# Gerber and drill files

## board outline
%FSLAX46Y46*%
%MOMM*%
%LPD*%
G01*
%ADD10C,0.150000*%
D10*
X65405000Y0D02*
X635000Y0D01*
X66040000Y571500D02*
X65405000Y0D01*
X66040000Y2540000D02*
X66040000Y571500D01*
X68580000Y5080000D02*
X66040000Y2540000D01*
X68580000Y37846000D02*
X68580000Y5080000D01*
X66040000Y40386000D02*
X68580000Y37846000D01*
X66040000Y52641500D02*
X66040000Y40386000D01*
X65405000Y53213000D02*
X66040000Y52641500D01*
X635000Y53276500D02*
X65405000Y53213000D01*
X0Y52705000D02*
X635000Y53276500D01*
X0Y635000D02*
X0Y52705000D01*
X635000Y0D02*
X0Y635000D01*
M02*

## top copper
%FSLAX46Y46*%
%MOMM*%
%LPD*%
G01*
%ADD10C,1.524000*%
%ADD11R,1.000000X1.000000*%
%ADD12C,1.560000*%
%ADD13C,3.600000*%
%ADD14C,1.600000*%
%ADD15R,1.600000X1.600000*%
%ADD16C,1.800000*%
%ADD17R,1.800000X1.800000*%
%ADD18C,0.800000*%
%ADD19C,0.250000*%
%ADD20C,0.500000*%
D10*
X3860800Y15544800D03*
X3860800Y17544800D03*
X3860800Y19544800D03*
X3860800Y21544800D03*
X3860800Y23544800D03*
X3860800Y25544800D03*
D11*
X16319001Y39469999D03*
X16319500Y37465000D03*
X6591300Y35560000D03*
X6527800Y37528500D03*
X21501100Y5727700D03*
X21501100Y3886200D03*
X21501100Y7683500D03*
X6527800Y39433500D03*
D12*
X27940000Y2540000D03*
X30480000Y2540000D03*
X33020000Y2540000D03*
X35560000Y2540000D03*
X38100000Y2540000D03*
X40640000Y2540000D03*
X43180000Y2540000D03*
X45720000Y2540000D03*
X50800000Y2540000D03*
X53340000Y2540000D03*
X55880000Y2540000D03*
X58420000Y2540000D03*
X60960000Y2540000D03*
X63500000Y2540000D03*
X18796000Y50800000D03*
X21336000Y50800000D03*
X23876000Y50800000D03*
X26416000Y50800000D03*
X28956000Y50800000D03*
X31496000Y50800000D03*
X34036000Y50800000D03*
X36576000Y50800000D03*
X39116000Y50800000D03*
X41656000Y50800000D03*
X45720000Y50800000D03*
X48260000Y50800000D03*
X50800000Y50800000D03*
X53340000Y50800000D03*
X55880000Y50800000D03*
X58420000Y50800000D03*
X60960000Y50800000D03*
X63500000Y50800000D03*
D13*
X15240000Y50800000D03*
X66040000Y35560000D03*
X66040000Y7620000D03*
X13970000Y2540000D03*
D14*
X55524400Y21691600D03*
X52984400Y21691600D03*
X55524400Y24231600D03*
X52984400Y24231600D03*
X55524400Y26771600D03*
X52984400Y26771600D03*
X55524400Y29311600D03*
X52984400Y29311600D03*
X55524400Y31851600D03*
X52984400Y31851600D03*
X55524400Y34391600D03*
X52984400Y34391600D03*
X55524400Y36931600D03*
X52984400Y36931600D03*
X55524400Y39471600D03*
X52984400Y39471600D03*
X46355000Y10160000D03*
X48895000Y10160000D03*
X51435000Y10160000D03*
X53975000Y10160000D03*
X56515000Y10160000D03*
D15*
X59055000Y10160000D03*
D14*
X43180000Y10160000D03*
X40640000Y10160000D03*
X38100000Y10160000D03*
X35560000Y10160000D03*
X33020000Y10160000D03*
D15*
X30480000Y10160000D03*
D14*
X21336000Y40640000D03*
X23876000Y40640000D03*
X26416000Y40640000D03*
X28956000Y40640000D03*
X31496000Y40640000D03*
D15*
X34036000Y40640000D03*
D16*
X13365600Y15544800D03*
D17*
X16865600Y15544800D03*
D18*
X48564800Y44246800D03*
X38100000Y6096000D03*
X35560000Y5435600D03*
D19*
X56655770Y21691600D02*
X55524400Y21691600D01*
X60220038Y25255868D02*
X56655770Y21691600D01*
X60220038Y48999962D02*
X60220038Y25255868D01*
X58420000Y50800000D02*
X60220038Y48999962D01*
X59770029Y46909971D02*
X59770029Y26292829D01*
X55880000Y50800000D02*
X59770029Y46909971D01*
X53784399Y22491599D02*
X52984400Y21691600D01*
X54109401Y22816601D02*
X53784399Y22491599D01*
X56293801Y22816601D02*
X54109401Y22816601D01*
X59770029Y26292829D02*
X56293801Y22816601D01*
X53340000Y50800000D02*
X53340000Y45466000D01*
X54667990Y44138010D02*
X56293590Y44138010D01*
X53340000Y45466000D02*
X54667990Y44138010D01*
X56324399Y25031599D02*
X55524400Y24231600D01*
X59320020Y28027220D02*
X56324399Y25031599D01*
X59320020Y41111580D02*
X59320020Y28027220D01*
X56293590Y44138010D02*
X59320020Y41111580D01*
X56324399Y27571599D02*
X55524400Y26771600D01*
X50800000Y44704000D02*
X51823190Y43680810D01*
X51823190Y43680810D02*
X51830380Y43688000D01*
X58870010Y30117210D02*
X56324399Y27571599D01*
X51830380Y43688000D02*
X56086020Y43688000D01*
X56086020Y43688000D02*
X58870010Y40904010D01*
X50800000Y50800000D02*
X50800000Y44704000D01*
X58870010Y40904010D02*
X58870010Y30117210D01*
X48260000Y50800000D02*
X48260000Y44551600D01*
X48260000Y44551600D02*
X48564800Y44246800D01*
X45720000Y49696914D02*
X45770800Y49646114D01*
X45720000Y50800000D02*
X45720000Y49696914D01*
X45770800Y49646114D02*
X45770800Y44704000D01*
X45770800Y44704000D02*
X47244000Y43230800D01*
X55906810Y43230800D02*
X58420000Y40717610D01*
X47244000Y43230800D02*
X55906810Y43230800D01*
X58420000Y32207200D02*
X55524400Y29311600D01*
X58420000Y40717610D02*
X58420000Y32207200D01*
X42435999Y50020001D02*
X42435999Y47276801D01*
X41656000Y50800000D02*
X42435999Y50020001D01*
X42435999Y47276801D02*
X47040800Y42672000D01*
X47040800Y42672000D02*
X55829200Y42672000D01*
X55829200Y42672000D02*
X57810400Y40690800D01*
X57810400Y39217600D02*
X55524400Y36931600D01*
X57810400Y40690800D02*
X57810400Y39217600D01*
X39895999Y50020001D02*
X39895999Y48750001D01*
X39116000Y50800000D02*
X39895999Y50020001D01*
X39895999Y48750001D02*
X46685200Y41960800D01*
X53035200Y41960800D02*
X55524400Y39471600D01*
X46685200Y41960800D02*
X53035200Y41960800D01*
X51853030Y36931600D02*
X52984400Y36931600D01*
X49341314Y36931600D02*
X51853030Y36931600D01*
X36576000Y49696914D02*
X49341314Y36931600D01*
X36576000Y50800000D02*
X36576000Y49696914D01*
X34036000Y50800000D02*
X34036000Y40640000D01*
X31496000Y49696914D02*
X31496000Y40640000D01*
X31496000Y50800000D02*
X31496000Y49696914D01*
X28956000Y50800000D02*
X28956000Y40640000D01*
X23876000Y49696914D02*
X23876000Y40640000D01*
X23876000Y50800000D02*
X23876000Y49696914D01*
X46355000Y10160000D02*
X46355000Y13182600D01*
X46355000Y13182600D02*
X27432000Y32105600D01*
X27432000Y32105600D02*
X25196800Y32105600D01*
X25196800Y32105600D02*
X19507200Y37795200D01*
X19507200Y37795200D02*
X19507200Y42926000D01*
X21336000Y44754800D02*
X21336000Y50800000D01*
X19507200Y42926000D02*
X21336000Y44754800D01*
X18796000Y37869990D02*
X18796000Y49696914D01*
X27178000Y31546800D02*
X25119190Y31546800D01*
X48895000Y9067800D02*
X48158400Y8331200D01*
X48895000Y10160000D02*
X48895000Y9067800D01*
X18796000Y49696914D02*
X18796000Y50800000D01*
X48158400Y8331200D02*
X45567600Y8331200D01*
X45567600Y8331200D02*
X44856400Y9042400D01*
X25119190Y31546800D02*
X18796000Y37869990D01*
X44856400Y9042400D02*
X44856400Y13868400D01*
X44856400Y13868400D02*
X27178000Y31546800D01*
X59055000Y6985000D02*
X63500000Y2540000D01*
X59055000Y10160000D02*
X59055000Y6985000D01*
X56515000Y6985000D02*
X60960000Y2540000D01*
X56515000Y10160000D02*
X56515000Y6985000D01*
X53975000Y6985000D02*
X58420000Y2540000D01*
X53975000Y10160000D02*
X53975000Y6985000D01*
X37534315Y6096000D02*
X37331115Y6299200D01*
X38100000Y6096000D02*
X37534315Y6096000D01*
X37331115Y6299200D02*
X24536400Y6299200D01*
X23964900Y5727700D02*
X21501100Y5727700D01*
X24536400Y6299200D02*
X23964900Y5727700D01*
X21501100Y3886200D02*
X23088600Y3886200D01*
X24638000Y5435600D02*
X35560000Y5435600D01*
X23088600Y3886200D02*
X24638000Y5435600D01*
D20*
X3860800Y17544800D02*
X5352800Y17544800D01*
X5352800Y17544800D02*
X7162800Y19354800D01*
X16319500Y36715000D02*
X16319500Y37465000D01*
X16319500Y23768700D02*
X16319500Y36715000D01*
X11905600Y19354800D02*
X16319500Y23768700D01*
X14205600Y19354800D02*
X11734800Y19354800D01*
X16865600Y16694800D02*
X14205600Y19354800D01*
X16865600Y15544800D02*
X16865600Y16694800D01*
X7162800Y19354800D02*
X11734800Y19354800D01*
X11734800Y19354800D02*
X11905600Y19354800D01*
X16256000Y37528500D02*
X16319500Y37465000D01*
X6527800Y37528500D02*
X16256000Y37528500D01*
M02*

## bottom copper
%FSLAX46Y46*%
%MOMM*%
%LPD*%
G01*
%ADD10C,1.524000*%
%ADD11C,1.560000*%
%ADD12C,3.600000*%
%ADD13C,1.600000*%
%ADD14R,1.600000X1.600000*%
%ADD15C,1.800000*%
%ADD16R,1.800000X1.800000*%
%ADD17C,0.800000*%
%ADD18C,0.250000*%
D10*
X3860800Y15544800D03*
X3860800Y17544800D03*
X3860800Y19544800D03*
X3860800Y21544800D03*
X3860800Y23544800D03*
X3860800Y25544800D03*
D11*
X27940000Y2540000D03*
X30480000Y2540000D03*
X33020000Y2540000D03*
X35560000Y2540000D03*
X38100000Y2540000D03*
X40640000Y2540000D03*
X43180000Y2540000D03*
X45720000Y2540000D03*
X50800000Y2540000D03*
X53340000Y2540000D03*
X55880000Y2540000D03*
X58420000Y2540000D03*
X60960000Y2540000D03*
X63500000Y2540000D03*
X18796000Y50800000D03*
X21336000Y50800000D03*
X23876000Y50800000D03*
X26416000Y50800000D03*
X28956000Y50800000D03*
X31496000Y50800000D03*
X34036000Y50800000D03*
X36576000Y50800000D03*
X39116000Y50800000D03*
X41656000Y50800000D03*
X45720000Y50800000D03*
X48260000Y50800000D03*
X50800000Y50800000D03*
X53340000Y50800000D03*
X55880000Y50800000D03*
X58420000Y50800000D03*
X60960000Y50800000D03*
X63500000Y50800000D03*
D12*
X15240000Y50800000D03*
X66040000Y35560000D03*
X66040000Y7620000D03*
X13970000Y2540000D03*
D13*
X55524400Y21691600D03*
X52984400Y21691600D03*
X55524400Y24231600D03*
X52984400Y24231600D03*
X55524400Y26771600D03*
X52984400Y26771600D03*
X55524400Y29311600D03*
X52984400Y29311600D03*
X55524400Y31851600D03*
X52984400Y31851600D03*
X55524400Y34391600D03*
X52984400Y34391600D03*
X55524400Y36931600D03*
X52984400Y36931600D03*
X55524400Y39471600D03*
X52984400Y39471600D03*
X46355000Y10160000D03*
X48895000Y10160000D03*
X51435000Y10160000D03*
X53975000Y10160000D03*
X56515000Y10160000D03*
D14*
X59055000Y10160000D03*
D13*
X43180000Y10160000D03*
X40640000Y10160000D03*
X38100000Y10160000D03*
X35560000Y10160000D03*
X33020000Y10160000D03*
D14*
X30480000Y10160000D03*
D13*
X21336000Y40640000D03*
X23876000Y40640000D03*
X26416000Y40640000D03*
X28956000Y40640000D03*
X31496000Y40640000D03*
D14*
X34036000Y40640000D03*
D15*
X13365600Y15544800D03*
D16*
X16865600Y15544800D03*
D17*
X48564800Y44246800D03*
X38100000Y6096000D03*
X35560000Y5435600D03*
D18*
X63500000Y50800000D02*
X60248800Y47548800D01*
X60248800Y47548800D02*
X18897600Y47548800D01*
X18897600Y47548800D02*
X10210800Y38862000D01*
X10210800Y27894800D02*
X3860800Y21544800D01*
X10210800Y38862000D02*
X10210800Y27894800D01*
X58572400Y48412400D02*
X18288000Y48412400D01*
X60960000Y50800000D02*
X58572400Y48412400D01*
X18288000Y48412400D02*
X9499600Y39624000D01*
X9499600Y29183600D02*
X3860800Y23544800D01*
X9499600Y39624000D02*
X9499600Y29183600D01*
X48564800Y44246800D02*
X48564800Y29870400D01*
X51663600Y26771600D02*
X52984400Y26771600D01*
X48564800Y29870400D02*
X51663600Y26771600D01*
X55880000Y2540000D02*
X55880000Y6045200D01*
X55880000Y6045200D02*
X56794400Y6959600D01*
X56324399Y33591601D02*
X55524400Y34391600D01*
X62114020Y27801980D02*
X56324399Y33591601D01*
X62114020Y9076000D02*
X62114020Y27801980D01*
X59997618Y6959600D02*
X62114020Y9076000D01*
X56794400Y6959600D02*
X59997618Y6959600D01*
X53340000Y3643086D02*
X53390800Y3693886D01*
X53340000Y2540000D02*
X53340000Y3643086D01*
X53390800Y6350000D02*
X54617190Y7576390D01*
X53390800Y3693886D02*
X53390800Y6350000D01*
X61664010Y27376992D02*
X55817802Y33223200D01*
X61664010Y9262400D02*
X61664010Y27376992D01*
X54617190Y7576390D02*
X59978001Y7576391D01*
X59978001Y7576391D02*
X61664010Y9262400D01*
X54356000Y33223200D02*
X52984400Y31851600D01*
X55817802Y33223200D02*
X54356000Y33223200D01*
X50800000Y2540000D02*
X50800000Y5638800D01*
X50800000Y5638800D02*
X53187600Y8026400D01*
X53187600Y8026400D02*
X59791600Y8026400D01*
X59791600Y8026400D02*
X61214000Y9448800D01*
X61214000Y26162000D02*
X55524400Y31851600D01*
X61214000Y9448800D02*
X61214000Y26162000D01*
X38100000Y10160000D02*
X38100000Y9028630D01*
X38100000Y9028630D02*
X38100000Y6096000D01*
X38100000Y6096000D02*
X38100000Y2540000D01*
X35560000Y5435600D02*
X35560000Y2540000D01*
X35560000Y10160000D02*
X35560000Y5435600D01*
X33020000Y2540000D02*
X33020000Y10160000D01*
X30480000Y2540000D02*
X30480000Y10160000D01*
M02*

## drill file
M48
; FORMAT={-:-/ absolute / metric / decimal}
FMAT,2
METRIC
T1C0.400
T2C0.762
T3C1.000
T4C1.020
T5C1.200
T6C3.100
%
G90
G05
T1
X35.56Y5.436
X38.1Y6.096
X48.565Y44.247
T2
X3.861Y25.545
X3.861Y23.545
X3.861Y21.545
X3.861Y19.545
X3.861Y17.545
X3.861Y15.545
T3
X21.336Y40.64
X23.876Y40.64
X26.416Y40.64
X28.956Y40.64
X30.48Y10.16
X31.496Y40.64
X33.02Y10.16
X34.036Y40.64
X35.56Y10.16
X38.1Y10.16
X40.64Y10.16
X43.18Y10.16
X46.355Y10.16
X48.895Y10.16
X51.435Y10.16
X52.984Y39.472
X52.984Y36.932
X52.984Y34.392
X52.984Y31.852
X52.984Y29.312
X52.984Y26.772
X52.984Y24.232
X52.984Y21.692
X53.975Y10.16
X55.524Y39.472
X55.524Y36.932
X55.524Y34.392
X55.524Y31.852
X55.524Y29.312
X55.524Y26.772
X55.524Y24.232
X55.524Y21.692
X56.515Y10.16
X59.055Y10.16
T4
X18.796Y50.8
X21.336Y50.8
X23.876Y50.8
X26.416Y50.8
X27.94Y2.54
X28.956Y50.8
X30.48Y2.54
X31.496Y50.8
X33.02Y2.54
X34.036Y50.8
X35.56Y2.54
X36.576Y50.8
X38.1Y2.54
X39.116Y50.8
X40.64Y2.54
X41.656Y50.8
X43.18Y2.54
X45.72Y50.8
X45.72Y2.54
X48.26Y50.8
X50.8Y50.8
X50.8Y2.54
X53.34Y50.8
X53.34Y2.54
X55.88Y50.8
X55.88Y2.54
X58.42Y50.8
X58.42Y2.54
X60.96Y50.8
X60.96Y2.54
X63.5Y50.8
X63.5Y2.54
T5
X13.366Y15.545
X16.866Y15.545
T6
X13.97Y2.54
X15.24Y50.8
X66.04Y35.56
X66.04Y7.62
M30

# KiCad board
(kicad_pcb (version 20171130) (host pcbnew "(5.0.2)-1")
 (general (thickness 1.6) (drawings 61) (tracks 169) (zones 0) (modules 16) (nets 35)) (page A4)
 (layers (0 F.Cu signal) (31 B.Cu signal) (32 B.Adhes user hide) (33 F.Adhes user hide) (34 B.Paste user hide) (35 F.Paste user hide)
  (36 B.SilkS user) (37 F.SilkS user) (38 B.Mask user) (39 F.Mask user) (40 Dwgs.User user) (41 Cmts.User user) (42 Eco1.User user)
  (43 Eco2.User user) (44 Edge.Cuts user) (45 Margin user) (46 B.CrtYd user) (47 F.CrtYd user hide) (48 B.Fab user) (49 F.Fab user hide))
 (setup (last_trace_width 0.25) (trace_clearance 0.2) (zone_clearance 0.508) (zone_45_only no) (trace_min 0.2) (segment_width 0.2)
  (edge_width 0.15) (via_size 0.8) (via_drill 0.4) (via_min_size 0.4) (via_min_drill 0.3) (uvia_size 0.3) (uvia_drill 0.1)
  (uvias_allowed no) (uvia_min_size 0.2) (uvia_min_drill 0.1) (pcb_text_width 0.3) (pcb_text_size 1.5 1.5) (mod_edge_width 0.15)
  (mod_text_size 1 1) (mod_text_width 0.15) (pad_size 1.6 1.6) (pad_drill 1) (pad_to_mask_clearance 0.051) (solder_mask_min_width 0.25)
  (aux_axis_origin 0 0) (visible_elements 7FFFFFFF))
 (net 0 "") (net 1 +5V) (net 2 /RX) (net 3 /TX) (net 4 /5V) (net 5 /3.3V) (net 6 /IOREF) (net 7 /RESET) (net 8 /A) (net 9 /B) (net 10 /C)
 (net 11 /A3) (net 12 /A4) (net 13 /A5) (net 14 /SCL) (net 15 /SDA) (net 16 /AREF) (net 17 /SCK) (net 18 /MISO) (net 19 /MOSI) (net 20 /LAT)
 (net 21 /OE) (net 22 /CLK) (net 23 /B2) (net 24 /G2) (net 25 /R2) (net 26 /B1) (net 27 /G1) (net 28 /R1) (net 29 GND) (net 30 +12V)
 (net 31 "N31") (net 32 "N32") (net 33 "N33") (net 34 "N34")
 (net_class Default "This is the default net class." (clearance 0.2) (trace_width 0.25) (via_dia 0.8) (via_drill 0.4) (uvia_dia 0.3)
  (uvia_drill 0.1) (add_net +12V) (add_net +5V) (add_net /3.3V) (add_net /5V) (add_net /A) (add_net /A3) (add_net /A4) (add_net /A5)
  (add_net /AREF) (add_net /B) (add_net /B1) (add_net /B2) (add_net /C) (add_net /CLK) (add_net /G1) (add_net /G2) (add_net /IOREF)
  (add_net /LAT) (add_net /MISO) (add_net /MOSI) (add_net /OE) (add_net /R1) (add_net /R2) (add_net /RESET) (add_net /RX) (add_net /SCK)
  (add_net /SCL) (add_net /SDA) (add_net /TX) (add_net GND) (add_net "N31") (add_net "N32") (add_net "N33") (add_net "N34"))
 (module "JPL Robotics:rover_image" (layer F.Cu) (at 38.4556 -27.7368 90)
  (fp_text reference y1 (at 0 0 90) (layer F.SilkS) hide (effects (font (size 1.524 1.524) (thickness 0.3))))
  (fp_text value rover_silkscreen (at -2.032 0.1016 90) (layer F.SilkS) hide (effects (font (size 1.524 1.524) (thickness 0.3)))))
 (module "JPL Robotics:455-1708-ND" (layer F.Cu) (at 3.8608 -15.5448 90)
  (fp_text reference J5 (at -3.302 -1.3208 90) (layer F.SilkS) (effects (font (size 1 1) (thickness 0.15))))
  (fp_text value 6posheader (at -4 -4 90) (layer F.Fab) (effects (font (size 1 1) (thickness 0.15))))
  (pad 1 thru_hole circle (at 0 0 90) (size 1.524 1.524) (drill 0.762) (layers *.Cu *.Mask))
  (pad 2 thru_hole circle (at 2 0 90) (size 1.524 1.524) (drill 0.762) (layers *.Cu *.Mask) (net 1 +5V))
  (pad 3 thru_hole circle (at 4 0 90) (size 1.524 1.524) (drill 0.762) (layers *.Cu *.Mask))
  (pad 4 thru_hole circle (at 6 0 90) (size 1.524 1.524) (drill 0.762) (layers *.Cu *.Mask) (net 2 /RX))
  (pad 5 thru_hole circle (at 8 0 90) (size 1.524 1.524) (drill 0.762) (layers *.Cu *.Mask) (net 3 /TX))
  (pad 6 thru_hole circle (at 10 0 90) (size 1.524 1.524) (drill 0.762) (layers *.Cu *.Mask)))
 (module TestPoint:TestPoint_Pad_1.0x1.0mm (layer F.Cu) (at 16.319001 -39.469999)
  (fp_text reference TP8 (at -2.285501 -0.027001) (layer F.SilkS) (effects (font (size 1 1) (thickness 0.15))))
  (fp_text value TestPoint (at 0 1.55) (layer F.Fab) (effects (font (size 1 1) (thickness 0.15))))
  (pad 1 smd rect (at 0 0) (size 1 1) (layers F.Cu F.Mask)))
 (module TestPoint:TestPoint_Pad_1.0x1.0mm (layer F.Cu) (at 16.3195 -37.465)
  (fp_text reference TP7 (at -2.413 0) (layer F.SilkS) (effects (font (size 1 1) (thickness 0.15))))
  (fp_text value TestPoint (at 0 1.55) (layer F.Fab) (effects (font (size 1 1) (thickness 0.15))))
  (pad 1 smd rect (at 0 0) (size 1 1) (layers F.Cu F.Mask) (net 1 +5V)))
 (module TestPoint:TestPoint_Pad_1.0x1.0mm (layer F.Cu) (at 6.5913 -35.56)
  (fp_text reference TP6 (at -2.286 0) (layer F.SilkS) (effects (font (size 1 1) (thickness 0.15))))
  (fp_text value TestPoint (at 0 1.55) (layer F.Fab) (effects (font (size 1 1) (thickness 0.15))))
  (pad 1 smd rect (at 0 0) (size 1 1) (layers F.Cu F.Mask)))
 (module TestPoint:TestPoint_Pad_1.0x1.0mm (layer F.Cu) (at 6.5278 -37.5285)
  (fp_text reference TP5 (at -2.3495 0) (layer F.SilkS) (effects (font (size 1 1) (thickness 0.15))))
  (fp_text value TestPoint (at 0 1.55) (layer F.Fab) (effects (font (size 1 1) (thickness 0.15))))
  (pad 1 smd rect (at 0 0) (size 1 1) (layers F.Cu F.Mask) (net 1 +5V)))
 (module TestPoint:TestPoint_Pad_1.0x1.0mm (layer F.Cu) (at 21.5011 -5.7277 90)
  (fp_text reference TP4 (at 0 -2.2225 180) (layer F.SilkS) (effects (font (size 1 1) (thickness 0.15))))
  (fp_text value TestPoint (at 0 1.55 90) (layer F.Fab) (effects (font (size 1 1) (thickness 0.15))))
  (pad 1 smd rect (at 0 0 90) (size 1 1) (layers F.Cu F.Mask) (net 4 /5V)))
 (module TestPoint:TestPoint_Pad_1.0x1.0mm (layer F.Cu) (at 21.5011 -3.8862 90)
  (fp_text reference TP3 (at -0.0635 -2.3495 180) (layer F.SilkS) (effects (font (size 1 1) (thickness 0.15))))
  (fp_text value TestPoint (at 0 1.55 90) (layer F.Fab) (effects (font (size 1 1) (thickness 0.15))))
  (pad 1 smd rect (at 0 0 90) (size 1 1) (layers F.Cu F.Mask) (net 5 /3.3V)))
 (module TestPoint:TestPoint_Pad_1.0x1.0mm (layer F.Cu) (at 21.5011 -7.6835 90)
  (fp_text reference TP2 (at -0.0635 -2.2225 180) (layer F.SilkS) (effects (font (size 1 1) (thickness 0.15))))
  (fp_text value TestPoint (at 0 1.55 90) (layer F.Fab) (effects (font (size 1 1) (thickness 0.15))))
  (pad 1 smd rect (at 0 0 90) (size 1 1) (layers F.Cu F.Mask)))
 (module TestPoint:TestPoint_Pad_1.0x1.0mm (layer F.Cu) (at 6.5278 -39.4335)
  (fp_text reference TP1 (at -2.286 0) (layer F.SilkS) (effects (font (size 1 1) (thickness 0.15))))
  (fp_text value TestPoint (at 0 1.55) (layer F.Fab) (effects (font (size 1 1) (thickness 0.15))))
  (pad 1 smd rect (at 0 0) (size 1 1) (layers F.Cu F.Mask)))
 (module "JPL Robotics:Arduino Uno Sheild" (layer F.Cu) (at 0 0)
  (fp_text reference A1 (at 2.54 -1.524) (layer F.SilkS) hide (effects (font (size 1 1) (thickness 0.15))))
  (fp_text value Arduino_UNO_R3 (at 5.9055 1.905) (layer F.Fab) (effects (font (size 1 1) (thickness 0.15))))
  (pad 31 thru_hole circle (at 27.94 -2.54) (size 1.56 1.56) (drill 1.02) (layers *.Cu *.Mask))
  (pad 20 thru_hole circle (at 30.48 -2.54) (size 1.56 1.56) (drill 1.02) (layers *.Cu *.Mask) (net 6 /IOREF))
  (pad 21 thru_hole circle (at 33.02 -2.54) (size 1.56 1.56) (drill 1.02) (layers *.Cu *.Mask) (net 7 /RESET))
  (pad 22 thru_hole circle (at 35.56 -2.54) (size 1.56 1.56) (drill 1.02) (layers *.Cu *.Mask) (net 5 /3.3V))
  (pad 23 thru_hole circle (at 38.1 -2.54) (size 1.56 1.56) (drill 1.02) (layers *.Cu *.Mask) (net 4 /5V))
  (pad 24 thru_hole circle (at 40.64 -2.54) (size 1.56 1.56) (drill 1.02) (layers *.Cu *.Mask))
  (pad 25 thru_hole circle (at 43.18 -2.54) (size 1.56 1.56) (drill 1.02) (layers *.Cu *.Mask))
  (pad 26 thru_hole circle (at 45.72 -2.54) (size 1.56 1.56) (drill 1.02) (layers *.Cu *.Mask))
  (pad 14 thru_hole circle (at 50.8 -2.54) (size 1.56 1.56) (drill 1.02) (layers *.Cu *.Mask) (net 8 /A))
  (pad 15 thru_hole circle (at 53.34 -2.54) (size 1.56 1.56) (drill 1.02) (layers *.Cu *.Mask) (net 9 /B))
  (pad 16 thru_hole circle (at 55.88 -2.54) (size 1.56 1.56) (drill 1.02) (layers *.Cu *.Mask) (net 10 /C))
  (pad 17 thru_hole circle (at 58.42 -2.54) (size 1.56 1.56) (drill 1.02) (layers *.Cu *.Mask) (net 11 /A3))
  (pad 18 thru_hole circle (at 60.96 -2.54) (size 1.56 1.56) (drill 1.02) (layers *.Cu *.Mask) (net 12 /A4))
  (pad 19 thru_hole circle (at 63.5 -2.54) (size 1.56 1.56) (drill 1.02) (layers *.Cu *.Mask) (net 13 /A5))
  (pad 30 thru_hole circle (at 18.796 -50.8) (size 1.56 1.56) (drill 1.02) (layers *.Cu *.Mask) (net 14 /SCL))
  (pad 29 thru_hole circle (at 21.336 -50.8) (size 1.56 1.56) (drill 1.02) (layers *.Cu *.Mask) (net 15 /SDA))
  (pad 28 thru_hole circle (at 23.876 -50.8) (size 1.56 1.56) (drill 1.02) (layers *.Cu *.Mask) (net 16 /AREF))
  (pad 27 thru_hole circle (at 26.416 -50.8) (size 1.56 1.56) (drill 1.02) (layers *.Cu *.Mask))
  (pad 13 thru_hole circle (at 28.956 -50.8) (size 1.56 1.56) (drill 1.02) (layers *.Cu *.Mask) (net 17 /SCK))
  (pad 12 thru_hole circle (at 31.496 -50.8) (size 1.56 1.56) (drill 1.02) (layers *.Cu *.Mask) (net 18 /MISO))
  (pad 11 thru_hole circle (at 34.036 -50.8) (size 1.56 1.56) (drill 1.02) (layers *.Cu *.Mask) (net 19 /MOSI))
  (pad 10 thru_hole circle (at 36.576 -50.8) (size 1.56 1.56) (drill 1.02) (layers *.Cu *.Mask) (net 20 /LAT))
  (pad 9 thru_hole circle (at 39.116 -50.8) (size 1.56 1.56) (drill 1.02) (layers *.Cu *.Mask) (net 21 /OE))
  (pad 8 thru_hole circle (at 41.656 -50.8) (size 1.56 1.56) (drill 1.02) (layers *.Cu *.Mask) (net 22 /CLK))
  (pad 7 thru_hole circle (at 45.72 -50.8) (size 1.56 1.56) (drill 1.02) (layers *.Cu *.Mask) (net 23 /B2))
  (pad 6 thru_hole circle (at 48.26 -50.8) (size 1.56 1.56) (drill 1.02) (layers *.Cu *.Mask) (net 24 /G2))
  (pad 5 thru_hole circle (at 50.8 -50.8) (size 1.56 1.56) (drill 1.02) (layers *.Cu *.Mask) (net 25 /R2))
  (pad 4 thru_hole circle (at 53.34 -50.8) (size 1.56 1.56) (drill 1.02) (layers *.Cu *.Mask) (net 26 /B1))
  (pad 3 thru_hole circle (at 55.88 -50.8) (size 1.56 1.56) (drill 1.02) (layers *.Cu *.Mask) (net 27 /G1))
  (pad 2 thru_hole circle (at 58.42 -50.8) (size 1.56 1.56) (drill 1.02) (layers *.Cu *.Mask) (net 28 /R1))
  (pad 1 thru_hole circle (at 60.96 -50.8) (size 1.56 1.56) (drill 1.02) (layers *.Cu *.Mask) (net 3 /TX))
  (pad 0 thru_hole circle (at 63.5 -50.8) (size 1.56 1.56) (drill 1.02) (layers *.Cu *.Mask) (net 2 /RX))
  (pad "" np_thru_hole circle (at 15.24 -50.8) (size 3.6 3.6) (drill 3.1) (layers *.Cu *.Mask))
  (pad "" np_thru_hole circle (at 66.04 -35.56) (size 3.6 3.6) (drill 3.1) (layers *.Cu *.Mask))
  (pad "" np_thru_hole circle (at 66.04 -7.62) (size 3.6 3.6) (drill 3.1) (layers *.Cu *.Mask))
  (pad "" np_thru_hole circle (at 13.97 -2.54) (size 3.6 3.6) (drill 3.1) (layers *.Cu *.Mask)))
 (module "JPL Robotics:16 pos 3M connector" (layer F.Cu) (at 54.2544 -30.5816 90)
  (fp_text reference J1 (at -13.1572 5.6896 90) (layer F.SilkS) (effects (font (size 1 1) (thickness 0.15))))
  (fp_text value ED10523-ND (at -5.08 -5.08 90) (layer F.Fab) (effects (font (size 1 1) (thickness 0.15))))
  (pad 1 thru_hole circle (at -8.89 1.27 90) (size 1.6 1.6) (drill 1) (layers *.Cu *.Mask) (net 28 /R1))
  (pad 2 thru_hole circle (at -8.89 -1.27 90) (size 1.6 1.6) (drill 1) (layers *.Cu *.Mask) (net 27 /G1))
  (pad 3 thru_hole circle (at -6.35 1.27 90) (size 1.6 1.6) (drill 1) (layers *.Cu *.Mask) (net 26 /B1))
  (pad 4 thru_hole circle (at -6.35 -1.27 90) (size 1.6 1.6) (drill 1) (layers *.Cu *.Mask))
  (pad 5 thru_hole circle (at -3.81 1.27 90) (size 1.6 1.6) (drill 1) (layers *.Cu *.Mask) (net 25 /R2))
  (pad 6 thru_hole circle (at -3.81 -1.27 90) (size 1.6 1.6) (drill 1) (layers *.Cu *.Mask) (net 24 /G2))
  (pad 7 thru_hole circle (at -1.27 1.27 90) (size 1.6 1.6) (drill 1) (layers *.Cu *.Mask) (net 23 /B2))
  (pad 8 thru_hole circle (at -1.27 -1.27 90) (size 1.6 1.6) (drill 1) (layers *.Cu *.Mask))
  (pad 9 thru_hole circle (at 1.27 1.27 90) (size 1.6 1.6) (drill 1) (layers *.Cu *.Mask) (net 8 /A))
  (pad 10 thru_hole circle (at 1.27 -1.27 90) (size 1.6 1.6) (drill 1) (layers *.Cu *.Mask) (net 9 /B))
  (pad 11 thru_hole circle (at 3.81 1.27 90) (size 1.6 1.6) (drill 1) (layers *.Cu *.Mask) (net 10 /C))
  (pad 12 thru_hole circle (at 3.81 -1.27 90) (size 1.6 1.6) (drill 1) (layers *.Cu *.Mask))
  (pad 13 thru_hole circle (at 6.35 1.27 90) (size 1.6 1.6) (drill 1) (layers *.Cu *.Mask) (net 22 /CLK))
  (pad 14 thru_hole circle (at 6.35 -1.27 90) (size 1.6 1.6) (drill 1) (layers *.Cu *.Mask) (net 20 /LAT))
  (pad 15 thru_hole circle (at 8.89 1.27 90) (size 1.6 1.6) (drill 1) (layers *.Cu *.Mask) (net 21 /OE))
  (pad 16 thru_hole circle (at 8.89 -1.27 90) (size 1.6 1.6) (drill 1) (layers *.Cu *.Mask)))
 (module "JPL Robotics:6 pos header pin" (layer F.Cu) (at 59.055 -10.16 180)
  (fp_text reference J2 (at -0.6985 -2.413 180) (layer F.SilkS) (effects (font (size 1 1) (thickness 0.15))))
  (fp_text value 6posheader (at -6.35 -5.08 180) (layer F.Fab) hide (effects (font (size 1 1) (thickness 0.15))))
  (pad 6 thru_hole circle (at 12.7 0 180) (size 1.6 1.6) (drill 1) (layers *.Cu *.Mask) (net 15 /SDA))
  (pad 5 thru_hole circle (at 10.16 0 180) (size 1.6 1.6) (drill 1) (layers *.Cu *.Mask) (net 14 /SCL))
  (pad 4 thru_hole circle (at 7.62 0 180) (size 1.6 1.6) (drill 1) (layers *.Cu *.Mask))
  (pad 3 thru_hole circle (at 5.08 0 180) (size 1.6 1.6) (drill 1) (layers *.Cu *.Mask) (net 11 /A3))
  (pad 2 thru_hole circle (at 2.54 0 180) (size 1.6 1.6) (drill 1) (layers *.Cu *.Mask) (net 12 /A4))
  (pad 1 thru_hole rect (at 0 0 180) (size 1.6 1.6) (drill 1) (layers *.Cu *.Mask) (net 13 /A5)))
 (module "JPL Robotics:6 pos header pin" (layer F.Cu) (at 30.48 -10.16)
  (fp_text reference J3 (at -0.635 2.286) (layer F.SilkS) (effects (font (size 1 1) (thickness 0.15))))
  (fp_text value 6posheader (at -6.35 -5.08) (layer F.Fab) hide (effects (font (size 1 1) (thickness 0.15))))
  (pad 6 thru_hole circle (at 12.7 0) (size 1.6 1.6) (drill 1) (layers *.Cu *.Mask))
  (pad 5 thru_hole circle (at 10.16 0) (size 1.6 1.6) (drill 1) (layers *.Cu *.Mask))
  (pad 4 thru_hole circle (at 7.62 0) (size 1.6 1.6) (drill 1) (layers *.Cu *.Mask) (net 4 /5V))
  (pad 3 thru_hole circle (at 5.08 0) (size 1.6 1.6) (drill 1) (layers *.Cu *.Mask) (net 5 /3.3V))
  (pad 2 thru_hole circle (at 2.54 0) (size 1.6 1.6) (drill 1) (layers *.Cu *.Mask) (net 7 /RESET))
  (pad 1 thru_hole rect (at 0 0) (size 1.6 1.6) (drill 1) (layers *.Cu *.Mask) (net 6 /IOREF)))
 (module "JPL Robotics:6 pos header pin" (layer F.Cu) (at 34.036 -40.64 180)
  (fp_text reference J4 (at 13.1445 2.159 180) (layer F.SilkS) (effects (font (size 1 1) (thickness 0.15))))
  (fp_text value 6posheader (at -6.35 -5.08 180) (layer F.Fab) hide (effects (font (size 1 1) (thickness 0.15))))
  (pad 6 thru_hole circle (at 12.7 0 180) (size 1.6 1.6) (drill 1) (layers *.Cu *.Mask))
  (pad 5 thru_hole circle (at 10.16 0 180) (size 1.6 1.6) (drill 1) (layers *.Cu *.Mask) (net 16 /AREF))
  (pad 4 thru_hole circle (at 7.62 0 180) (size 1.6 1.6) (drill 1) (layers *.Cu *.Mask))
  (pad 3 thru_hole circle (at 5.08 0 180) (size 1.6 1.6) (drill 1) (layers *.Cu *.Mask) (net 17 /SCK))
  (pad 2 thru_hole circle (at 2.54 0 180) (size 1.6 1.6) (drill 1) (layers *.Cu *.Mask) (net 18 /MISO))
  (pad 1 thru_hole rect (at 0 0 180) (size 1.6 1.6) (drill 1) (layers *.Cu *.Mask) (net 19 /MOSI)))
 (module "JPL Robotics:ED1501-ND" (layer F.Cu) (at 16.8656 -15.5448 180)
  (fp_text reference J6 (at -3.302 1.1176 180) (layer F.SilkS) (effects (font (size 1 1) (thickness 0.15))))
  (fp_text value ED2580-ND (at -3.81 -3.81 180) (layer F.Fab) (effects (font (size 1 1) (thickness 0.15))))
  (pad 2 thru_hole circle (at 3.5 0 180) (size 1.8 1.8) (drill 1.2) (layers *.Cu *.Mask))
  (pad 1 thru_hole rect (at 0 0 180) (size 1.8 1.8) (drill 1.2) (layers *.Cu *.Mask) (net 1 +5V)))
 (gr_line (start 65.405 0) (end 0.635 0) (layer Edge.Cuts) (width 0.15))
 (gr_line (start 66.04 -0.5715) (end 65.405 0) (layer Edge.Cuts) (width 0.15))
 (gr_line (start 66.04 -2.54) (end 66.04 -0.5715) (layer Edge.Cuts) (width 0.15))
 (gr_line (start 68.58 -5.08) (end 66.04 -2.54) (layer Edge.Cuts) (width 0.15))
 (gr_line (start 68.58 -37.846) (end 68.58 -5.08) (layer Edge.Cuts) (width 0.15))
 (gr_line (start 66.04 -40.386) (end 68.58 -37.846) (layer Edge.Cuts) (width 0.15))
 (gr_line (start 66.04 -52.6415) (end 66.04 -40.386) (layer Edge.Cuts) (width 0.15))
 (gr_line (start 65.405 -53.213) (end 66.04 -52.6415) (layer Edge.Cuts) (width 0.15))
 (gr_line (start 0.635 -53.2765) (end 65.405 -53.213) (layer Edge.Cuts) (width 0.15))
 (gr_line (start 0 -52.705) (end 0.635 -53.2765) (layer Edge.Cuts) (width 0.15))
 (gr_line (start 0 -0.635) (end 0 -52.705) (layer Edge.Cuts) (width 0.15))
 (gr_line (start 0.635 0) (end 0 -0.635) (layer Edge.Cuts) (width 0.15))
 (segment (start 63.5 -50.8) (end 60.2488 -47.5488) (width 0.25) (layer B.Cu) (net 2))
 (segment (start 60.2488 -47.5488) (end 18.8976 -47.5488) (width 0.25) (layer B.Cu) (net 2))
 (segment (start 18.8976 -47.5488) (end 10.2108 -38.862) (width 0.25) (layer B.Cu) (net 2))
 (segment (start 10.2108 -27.8948) (end 3.8608 -21.5448) (width 0.25) (layer B.Cu) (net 2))
 (segment (start 10.2108 -38.862) (end 10.2108 -27.8948) (width 0.25) (layer B.Cu) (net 2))
 (segment (start 58.5724 -48.4124) (end 18.288 -48.4124) (width 0.25) (layer B.Cu) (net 3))
 (segment (start 60.96 -50.8) (end 58.5724 -48.4124) (width 0.25) (layer B.Cu) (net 3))
 (segment (start 18.288 -48.4124) (end 9.4996 -39.624) (width 0.25) (layer B.Cu) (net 3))
 (segment (start 9.4996 -29.1836) (end 3.8608 -23.5448) (width 0.25) (layer B.Cu) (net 3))
 (segment (start 9.4996 -39.624) (end 9.4996 -29.1836) (width 0.25) (layer B.Cu) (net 3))
 (segment (start 56.65577 -21.6916) (end 55.5244 -21.6916) (width 0.25) (layer F.Cu) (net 28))
 (segment (start 60.220038 -25.255868) (end 56.65577 -21.6916) (width 0.25) (layer F.Cu) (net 28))
 (segment (start 60.220038 -48.999962) (end 60.220038 -25.255868) (width 0.25) (layer F.Cu) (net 28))
 (segment (start 58.42 -50.8) (end 60.220038 -48.999962) (width 0.25) (layer F.Cu) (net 28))
 (segment (start 59.770029 -46.909971) (end 59.770029 -26.292829) (width 0.25) (layer F.Cu) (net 27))
 (segment (start 55.88 -50.8) (end 59.770029 -46.909971) (width 0.25) (layer F.Cu) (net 27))
 (segment (start 53.784399 -22.491599) (end 52.9844 -21.6916) (width 0.25) (layer F.Cu) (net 27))
 (segment (start 54.109401 -22.816601) (end 53.784399 -22.491599) (width 0.25) (layer F.Cu) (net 27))
 (segment (start 56.293801 -22.816601) (end 54.109401 -22.816601) (width 0.25) (layer F.Cu) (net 27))
 (segment (start 59.770029 -26.292829) (end 56.293801 -22.816601) (width 0.25) (layer F.Cu) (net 27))
 (segment (start 53.34 -50.8) (end 53.34 -45.466) (width 0.25) (layer F.Cu) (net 26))
 (segment (start 54.66799 -44.13801) (end 56.29359 -44.13801) (width 0.25) (layer F.Cu) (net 26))
 (segment (start 53.34 -45.466) (end 54.66799 -44.13801) (width 0.25) (layer F.Cu) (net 26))
 (segment (start 56.324399 -25.031599) (end 55.5244 -24.2316) (width 0.25) (layer F.Cu) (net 26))
 (segment (start 59.32002 -28.02722) (end 56.324399 -25.031599) (width 0.25) (layer F.Cu) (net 26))
 (segment (start 59.32002 -41.11158) (end 59.32002 -28.02722) (width 0.25) (layer F.Cu) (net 26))
 (segment (start 56.29359 -44.13801) (end 59.32002 -41.11158) (width 0.25) (layer F.Cu) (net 26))
 (segment (start 56.324399 -27.571599) (end 55.5244 -26.7716) (width 0.25) (layer F.Cu) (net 25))
 (segment (start 50.8 -44.704) (end 51.82319 -43.68081) (width 0.25) (layer F.Cu) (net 25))
 (segment (start 51.82319 -43.68081) (end 51.83038 -43.688) (width 0.25) (layer F.Cu) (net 25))
 (segment (start 58.87001 -30.11721) (end 56.324399 -27.571599) (width 0.25) (layer F.Cu) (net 25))
 (segment (start 51.83038 -43.688) (end 56.08602 -43.688) (width 0.25) (layer F.Cu) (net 25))
 (segment (start 56.08602 -43.688) (end 58.87001 -40.90401) (width 0.25) (layer F.Cu) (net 25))
 (segment (start 50.8 -50.8) (end 50.8 -44.704) (width 0.25) (layer F.Cu) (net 25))
 (segment (start 58.87001 -40.90401) (end 58.87001 -30.11721) (width 0.25) (layer F.Cu) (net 25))
 (segment (start 48.26 -50.8) (end 48.26 -44.5516) (width 0.25) (layer F.Cu) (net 24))
 (segment (start 48.26 -44.5516) (end 48.5648 -44.2468) (width 0.25) (layer F.Cu) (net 24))
 (segment (start 48.5648 -44.2468) (end 48.5648 -29.8704) (width 0.25) (layer B.Cu) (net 24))
 (segment (start 51.6636 -26.7716) (end 52.9844 -26.7716) (width 0.25) (layer B.Cu) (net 24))
 (segment (start 48.5648 -29.8704) (end 51.6636 -26.7716) (width 0.25) (layer B.Cu) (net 24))
 (segment (start 45.72 -49.696914) (end 45.7708 -49.646114) (width 0.25) (layer F.Cu) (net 23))
 (segment (start 45.72 -50.8) (end 45.72 -49.696914) (width 0.25) (layer F.Cu) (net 23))
 (segment (start 45.7708 -49.646114) (end 45.7708 -44.704) (width 0.25) (layer F.Cu) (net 23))
 (segment (start 45.7708 -44.704) (end 47.244 -43.2308) (width 0.25) (layer F.Cu) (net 23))
 (segment (start 55.90681 -43.2308) (end 58.42 -40.71761) (width 0.25) (layer F.Cu) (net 23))
 (segment (start 47.244 -43.2308) (end 55.90681 -43.2308) (width 0.25) (layer F.Cu) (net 23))
 (segment (start 58.42 -32.2072) (end 55.5244 -29.3116) (width 0.25) (layer F.Cu) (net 23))
 (segment (start 58.42 -40.71761) (end 58.42 -32.2072) (width 0.25) (layer F.Cu) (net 23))
 (segment (start 42.435999 -50.020001) (end 42.435999 -47.276801) (width 0.25) (layer F.Cu) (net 22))
 (segment (start 41.656 -50.8) (end 42.435999 -50.020001) (width 0.25) (layer F.Cu) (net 22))
 (segment (start 42.435999 -47.276801) (end 47.0408 -42.672) (width 0.25) (layer F.Cu) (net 22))
 (segment (start 47.0408 -42.672) (end 55.8292 -42.672) (width 0.25) (layer F.Cu) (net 22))
 (segment (start 55.8292 -42.672) (end 57.8104 -40.6908) (width 0.25) (layer F.Cu) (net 22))
 (segment (start 57.8104 -39.2176) (end 55.5244 -36.9316) (width 0.25) (layer F.Cu) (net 22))
 (segment (start 57.8104 -40.6908) (end 57.8104 -39.2176) (width 0.25) (layer F.Cu) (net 22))
 (segment (start 39.895999 -50.020001) (end 39.895999 -48.750001) (width 0.25) (layer F.Cu) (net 21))
 (segment (start 39.116 -50.8) (end 39.895999 -50.020001) (width 0.25) (layer F.Cu) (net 21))
 (segment (start 39.895999 -48.750001) (end 46.6852 -41.9608) (width 0.25) (layer F.Cu) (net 21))
 (segment (start 53.0352 -41.9608) (end 55.5244 -39.4716) (width 0.25) (layer F.Cu) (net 21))
 (segment (start 46.6852 -41.9608) (end 53.0352 -41.9608) (width 0.25) (layer F.Cu) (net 21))
 (segment (start 51.85303 -36.9316) (end 52.9844 -36.9316) (width 0.25) (layer F.Cu) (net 20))
 (segment (start 49.341314 -36.9316) (end 51.85303 -36.9316) (width 0.25) (layer F.Cu) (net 20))
 (segment (start 36.576 -49.696914) (end 49.341314 -36.9316) (width 0.25) (layer F.Cu) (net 20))
 (segment (start 36.576 -50.8) (end 36.576 -49.696914) (width 0.25) (layer F.Cu) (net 20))
 (segment (start 34.036 -50.8) (end 34.036 -40.64) (width 0.25) (layer F.Cu) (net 19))
 (segment (start 31.496 -49.696914) (end 31.496 -40.64) (width 0.25) (layer F.Cu) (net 18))
 (segment (start 31.496 -50.8) (end 31.496 -49.696914) (width 0.25) (layer F.Cu) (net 18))
 (segment (start 28.956 -50.8) (end 28.956 -40.64) (width 0.25) (layer F.Cu) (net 17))
 (segment (start 23.876 -49.696914) (end 23.876 -40.64) (width 0.25) (layer F.Cu) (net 16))
 (segment (start 23.876 -50.8) (end 23.876 -49.696914) (width 0.25) (layer F.Cu) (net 16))
 (segment (start 46.355 -10.16) (end 46.355 -13.1826) (width 0.25) (layer F.Cu) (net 15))
 (segment (start 46.355 -13.1826) (end 27.432 -32.1056) (width 0.25) (layer F.Cu) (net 15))
 (segment (start 27.432 -32.1056) (end 25.1968 -32.1056) (width 0.25) (layer F.Cu) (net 15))
 (segment (start 25.1968 -32.1056) (end 19.5072 -37.7952) (width 0.25) (layer F.Cu) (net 15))
 (segment (start 19.5072 -37.7952) (end 19.5072 -42.926) (width 0.25) (layer F.Cu) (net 15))
 (segment (start 21.336 -44.7548) (end 21.336 -50.8) (width 0.25) (layer F.Cu) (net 15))
 (segment (start 19.5072 -42.926) (end 21.336 -44.7548) (width 0.25) (layer F.Cu) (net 15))
 (segment (start 18.796 -37.86999) (end 18.796 -49.696914) (width 0.25) (layer F.Cu) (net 14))
 (segment (start 27.178 -31.5468) (end 25.11919 -31.5468) (width 0.25) (layer F.Cu) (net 14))
 (segment (start 48.895 -9.0678) (end 48.1584 -8.3312) (width 0.25) (layer F.Cu) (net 14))
 (segment (start 48.895 -10.16) (end 48.895 -9.0678) (width 0.25) (layer F.Cu) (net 14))
 (segment (start 18.796 -49.696914) (end 18.796 -50.8) (width 0.25) (layer F.Cu) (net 14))
 (segment (start 48.1584 -8.3312) (end 45.5676 -8.3312) (width 0.25) (layer F.Cu) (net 14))
 (segment (start 45.5676 -8.3312) (end 44.8564 -9.0424) (width 0.25) (layer F.Cu) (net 14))
 (segment (start 25.11919 -31.5468) (end 18.796 -37.86999) (width 0.25) (layer F.Cu) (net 14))
 (segment (start 44.8564 -9.0424) (end 44.8564 -13.8684) (width 0.25) (layer F.Cu) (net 14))
 (segment (start 44.8564 -13.8684) (end 27.178 -31.5468) (width 0.25) (layer F.Cu) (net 14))
 (segment (start 59.055 -6.985) (end 63.5 -2.54) (width 0.25) (layer F.Cu) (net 13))
 (segment (start 59.055 -10.16) (end 59.055 -6.985) (width 0.25) (layer F.Cu) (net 13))
 (segment (start 56.515 -6.985) (end 60.96 -2.54) (width 0.25) (layer F.Cu) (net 12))
 (segment (start 56.515 -10.16) (end 56.515 -6.985) (width 0.25) (layer F.Cu) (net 12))
 (segment (start 53.975 -6.985) (end 58.42 -2.54) (width 0.25) (layer F.Cu) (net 11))
 (segment (start 53.975 -10.16) (end 53.975 -6.985) (width 0.25) (layer F.Cu) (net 11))
 (segment (start 55.88 -2.54) (end 55.88 -6.0452) (width 0.25) (layer B.Cu) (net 10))
 (segment (start 55.88 -6.0452) (end 56.7944 -6.9596) (width 0.25) (layer B.Cu) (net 10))
 (segment (start 56.324399 -33.591601) (end 55.5244 -34.3916) (width 0.25) (layer B.Cu) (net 10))
 (segment (start 62.11402 -27.80198) (end 56.324399 -33.591601) (width 0.25) (layer B.Cu) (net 10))
 (segment (start 62.11402 -9.076) (end 62.11402 -27.80198) (width 0.25) (layer B.Cu) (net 10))
 (segment (start 59.997618 -6.9596) (end 62.11402 -9.076) (width 0.25) (layer B.Cu) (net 10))
 (segment (start 56.7944 -6.9596) (end 59.997618 -6.9596) (width 0.25) (layer B.Cu) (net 10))
 (segment (start 53.34 -3.643086) (end 53.3908 -3.693886) (width 0.25) (layer B.Cu) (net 9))
 (segment (start 53.34 -2.54) (end 53.34 -3.643086) (width 0.25) (layer B.Cu) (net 9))
 (segment (start 53.3908 -6.35) (end 54.61719 -7.57639) (width 0.25) (layer B.Cu) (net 9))
 (segment (start 53.3908 -3.693886) (end 53.3908 -6.35) (width 0.25) (layer B.Cu) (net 9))
 (segment (start 61.66401 -27.376992) (end 55.817802 -33.2232) (width 0.25) (layer B.Cu) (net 9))
 (segment (start 61.66401 -9.2624) (end 61.66401 -27.376992) (width 0.25) (layer B.Cu) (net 9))
 (segment (start 54.61719 -7.57639) (end 59.978001 -7.576391) (width 0.25) (layer B.Cu) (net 9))
 (segment (start 59.978001 -7.576391) (end 61.66401 -9.2624) (width 0.25) (layer B.Cu) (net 9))
 (segment (start 54.356 -33.2232) (end 52.9844 -31.8516) (width 0.25) (layer B.Cu) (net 9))
 (segment (start 55.817802 -33.2232) (end 54.356 -33.2232) (width 0.25) (layer B.Cu) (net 9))
 (segment (start 50.8 -2.54) (end 50.8 -5.6388) (width 0.25) (layer B.Cu) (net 8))
 (segment (start 50.8 -5.6388) (end 53.1876 -8.0264) (width 0.25) (layer B.Cu) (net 8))
 (segment (start 53.1876 -8.0264) (end 59.7916 -8.0264) (width 0.25) (layer B.Cu) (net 8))
 (segment (start 59.7916 -8.0264) (end 61.214 -9.4488) (width 0.25) (layer B.Cu) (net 8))
 (segment (start 61.214 -26.162) (end 55.5244 -31.8516) (width 0.25) (layer B.Cu) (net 8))
 (segment (start 61.214 -9.4488) (end 61.214 -26.162) (width 0.25) (layer B.Cu) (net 8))
 (segment (start 38.1 -10.16) (end 38.1 -9.02863) (width 0.25) (layer B.Cu) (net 4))
 (segment (start 38.1 -9.02863) (end 38.1 -6.096) (width 0.25) (layer B.Cu) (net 4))
 (segment (start 38.1 -6.096) (end 38.1 -2.54) (width 0.25) (layer B.Cu) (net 4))
 (segment (start 37.534315 -6.096) (end 37.331115 -6.2992) (width 0.25) (layer F.Cu) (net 4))
 (segment (start 38.1 -6.096) (end 37.534315 -6.096) (width 0.25) (layer F.Cu) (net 4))
 (segment (start 37.331115 -6.2992) (end 24.5364 -6.2992) (width 0.25) (layer F.Cu) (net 4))
 (segment (start 23.9649 -5.7277) (end 21.5011 -5.7277) (width 0.25) (layer F.Cu) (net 4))
 (segment (start 24.5364 -6.2992) (end 23.9649 -5.7277) (width 0.25) (layer F.Cu) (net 4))
 (segment (start 35.56 -5.4356) (end 35.56 -2.54) (width 0.25) (layer B.Cu) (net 5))
 (segment (start 35.56 -10.16) (end 35.56 -5.4356) (width 0.25) (layer B.Cu) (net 5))
 (segment (start 21.5011 -3.8862) (end 23.0886 -3.8862) (width 0.25) (layer F.Cu) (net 5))
 (segment (start 24.638 -5.4356) (end 35.56 -5.4356) (width 0.25) (layer F.Cu) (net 5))
 (segment (start 23.0886 -3.8862) (end 24.638 -5.4356) (width 0.25) (layer F.Cu) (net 5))
 (segment (start 33.02 -2.54) (end 33.02 -10.16) (width 0.25) (layer B.Cu) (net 7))
 (segment (start 30.48 -2.54) (end 30.48 -10.16) (width 0.25) (layer B.Cu) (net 6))
 (segment (start 3.8608 -17.5448) (end 5.3528 -17.5448) (width 0.5) (layer F.Cu) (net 1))
 (segment (start 5.3528 -17.5448) (end 7.1628 -19.3548) (width 0.5) (layer F.Cu) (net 1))
 (segment (start 16.3195 -36.715) (end 16.3195 -37.465) (width 0.5) (layer F.Cu) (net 1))
 (segment (start 16.3195 -23.7687) (end 16.3195 -36.715) (width 0.5) (layer F.Cu) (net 1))
 (segment (start 11.9056 -19.3548) (end 16.3195 -23.7687) (width 0.5) (layer F.Cu) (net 1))
 (segment (start 14.2056 -19.3548) (end 11.7348 -19.3548) (width 0.5) (layer F.Cu) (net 1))
 (segment (start 16.8656 -16.6948) (end 14.2056 -19.3548) (width 0.5) (layer F.Cu) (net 1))
 (segment (start 16.8656 -15.5448) (end 16.8656 -16.6948) (width 0.5) (layer F.Cu) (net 1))
 (segment (start 7.1628 -19.3548) (end 11.7348 -19.3548) (width 0.5) (layer F.Cu) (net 1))
 (segment (start 11.7348 -19.3548) (end 11.9056 -19.3548) (width 0.5) (layer F.Cu) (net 1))
 (segment (start 16.256 -37.5285) (end 16.3195 -37.465) (width 0.5) (layer F.Cu) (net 1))
 (segment (start 6.5278 -37.5285) (end 16.256 -37.5285) (width 0.5) (layer F.Cu) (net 1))
 (via (at 48.5648 -44.2468) (size 0.8) (layers F.Cu B.Cu) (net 24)) (via (at 38.1 -6.096) (size 0.8) (layers F.Cu B.Cu) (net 4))
 (via (at 35.56 -5.4356) (size 0.8) (layers F.Cu B.Cu) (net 5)))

